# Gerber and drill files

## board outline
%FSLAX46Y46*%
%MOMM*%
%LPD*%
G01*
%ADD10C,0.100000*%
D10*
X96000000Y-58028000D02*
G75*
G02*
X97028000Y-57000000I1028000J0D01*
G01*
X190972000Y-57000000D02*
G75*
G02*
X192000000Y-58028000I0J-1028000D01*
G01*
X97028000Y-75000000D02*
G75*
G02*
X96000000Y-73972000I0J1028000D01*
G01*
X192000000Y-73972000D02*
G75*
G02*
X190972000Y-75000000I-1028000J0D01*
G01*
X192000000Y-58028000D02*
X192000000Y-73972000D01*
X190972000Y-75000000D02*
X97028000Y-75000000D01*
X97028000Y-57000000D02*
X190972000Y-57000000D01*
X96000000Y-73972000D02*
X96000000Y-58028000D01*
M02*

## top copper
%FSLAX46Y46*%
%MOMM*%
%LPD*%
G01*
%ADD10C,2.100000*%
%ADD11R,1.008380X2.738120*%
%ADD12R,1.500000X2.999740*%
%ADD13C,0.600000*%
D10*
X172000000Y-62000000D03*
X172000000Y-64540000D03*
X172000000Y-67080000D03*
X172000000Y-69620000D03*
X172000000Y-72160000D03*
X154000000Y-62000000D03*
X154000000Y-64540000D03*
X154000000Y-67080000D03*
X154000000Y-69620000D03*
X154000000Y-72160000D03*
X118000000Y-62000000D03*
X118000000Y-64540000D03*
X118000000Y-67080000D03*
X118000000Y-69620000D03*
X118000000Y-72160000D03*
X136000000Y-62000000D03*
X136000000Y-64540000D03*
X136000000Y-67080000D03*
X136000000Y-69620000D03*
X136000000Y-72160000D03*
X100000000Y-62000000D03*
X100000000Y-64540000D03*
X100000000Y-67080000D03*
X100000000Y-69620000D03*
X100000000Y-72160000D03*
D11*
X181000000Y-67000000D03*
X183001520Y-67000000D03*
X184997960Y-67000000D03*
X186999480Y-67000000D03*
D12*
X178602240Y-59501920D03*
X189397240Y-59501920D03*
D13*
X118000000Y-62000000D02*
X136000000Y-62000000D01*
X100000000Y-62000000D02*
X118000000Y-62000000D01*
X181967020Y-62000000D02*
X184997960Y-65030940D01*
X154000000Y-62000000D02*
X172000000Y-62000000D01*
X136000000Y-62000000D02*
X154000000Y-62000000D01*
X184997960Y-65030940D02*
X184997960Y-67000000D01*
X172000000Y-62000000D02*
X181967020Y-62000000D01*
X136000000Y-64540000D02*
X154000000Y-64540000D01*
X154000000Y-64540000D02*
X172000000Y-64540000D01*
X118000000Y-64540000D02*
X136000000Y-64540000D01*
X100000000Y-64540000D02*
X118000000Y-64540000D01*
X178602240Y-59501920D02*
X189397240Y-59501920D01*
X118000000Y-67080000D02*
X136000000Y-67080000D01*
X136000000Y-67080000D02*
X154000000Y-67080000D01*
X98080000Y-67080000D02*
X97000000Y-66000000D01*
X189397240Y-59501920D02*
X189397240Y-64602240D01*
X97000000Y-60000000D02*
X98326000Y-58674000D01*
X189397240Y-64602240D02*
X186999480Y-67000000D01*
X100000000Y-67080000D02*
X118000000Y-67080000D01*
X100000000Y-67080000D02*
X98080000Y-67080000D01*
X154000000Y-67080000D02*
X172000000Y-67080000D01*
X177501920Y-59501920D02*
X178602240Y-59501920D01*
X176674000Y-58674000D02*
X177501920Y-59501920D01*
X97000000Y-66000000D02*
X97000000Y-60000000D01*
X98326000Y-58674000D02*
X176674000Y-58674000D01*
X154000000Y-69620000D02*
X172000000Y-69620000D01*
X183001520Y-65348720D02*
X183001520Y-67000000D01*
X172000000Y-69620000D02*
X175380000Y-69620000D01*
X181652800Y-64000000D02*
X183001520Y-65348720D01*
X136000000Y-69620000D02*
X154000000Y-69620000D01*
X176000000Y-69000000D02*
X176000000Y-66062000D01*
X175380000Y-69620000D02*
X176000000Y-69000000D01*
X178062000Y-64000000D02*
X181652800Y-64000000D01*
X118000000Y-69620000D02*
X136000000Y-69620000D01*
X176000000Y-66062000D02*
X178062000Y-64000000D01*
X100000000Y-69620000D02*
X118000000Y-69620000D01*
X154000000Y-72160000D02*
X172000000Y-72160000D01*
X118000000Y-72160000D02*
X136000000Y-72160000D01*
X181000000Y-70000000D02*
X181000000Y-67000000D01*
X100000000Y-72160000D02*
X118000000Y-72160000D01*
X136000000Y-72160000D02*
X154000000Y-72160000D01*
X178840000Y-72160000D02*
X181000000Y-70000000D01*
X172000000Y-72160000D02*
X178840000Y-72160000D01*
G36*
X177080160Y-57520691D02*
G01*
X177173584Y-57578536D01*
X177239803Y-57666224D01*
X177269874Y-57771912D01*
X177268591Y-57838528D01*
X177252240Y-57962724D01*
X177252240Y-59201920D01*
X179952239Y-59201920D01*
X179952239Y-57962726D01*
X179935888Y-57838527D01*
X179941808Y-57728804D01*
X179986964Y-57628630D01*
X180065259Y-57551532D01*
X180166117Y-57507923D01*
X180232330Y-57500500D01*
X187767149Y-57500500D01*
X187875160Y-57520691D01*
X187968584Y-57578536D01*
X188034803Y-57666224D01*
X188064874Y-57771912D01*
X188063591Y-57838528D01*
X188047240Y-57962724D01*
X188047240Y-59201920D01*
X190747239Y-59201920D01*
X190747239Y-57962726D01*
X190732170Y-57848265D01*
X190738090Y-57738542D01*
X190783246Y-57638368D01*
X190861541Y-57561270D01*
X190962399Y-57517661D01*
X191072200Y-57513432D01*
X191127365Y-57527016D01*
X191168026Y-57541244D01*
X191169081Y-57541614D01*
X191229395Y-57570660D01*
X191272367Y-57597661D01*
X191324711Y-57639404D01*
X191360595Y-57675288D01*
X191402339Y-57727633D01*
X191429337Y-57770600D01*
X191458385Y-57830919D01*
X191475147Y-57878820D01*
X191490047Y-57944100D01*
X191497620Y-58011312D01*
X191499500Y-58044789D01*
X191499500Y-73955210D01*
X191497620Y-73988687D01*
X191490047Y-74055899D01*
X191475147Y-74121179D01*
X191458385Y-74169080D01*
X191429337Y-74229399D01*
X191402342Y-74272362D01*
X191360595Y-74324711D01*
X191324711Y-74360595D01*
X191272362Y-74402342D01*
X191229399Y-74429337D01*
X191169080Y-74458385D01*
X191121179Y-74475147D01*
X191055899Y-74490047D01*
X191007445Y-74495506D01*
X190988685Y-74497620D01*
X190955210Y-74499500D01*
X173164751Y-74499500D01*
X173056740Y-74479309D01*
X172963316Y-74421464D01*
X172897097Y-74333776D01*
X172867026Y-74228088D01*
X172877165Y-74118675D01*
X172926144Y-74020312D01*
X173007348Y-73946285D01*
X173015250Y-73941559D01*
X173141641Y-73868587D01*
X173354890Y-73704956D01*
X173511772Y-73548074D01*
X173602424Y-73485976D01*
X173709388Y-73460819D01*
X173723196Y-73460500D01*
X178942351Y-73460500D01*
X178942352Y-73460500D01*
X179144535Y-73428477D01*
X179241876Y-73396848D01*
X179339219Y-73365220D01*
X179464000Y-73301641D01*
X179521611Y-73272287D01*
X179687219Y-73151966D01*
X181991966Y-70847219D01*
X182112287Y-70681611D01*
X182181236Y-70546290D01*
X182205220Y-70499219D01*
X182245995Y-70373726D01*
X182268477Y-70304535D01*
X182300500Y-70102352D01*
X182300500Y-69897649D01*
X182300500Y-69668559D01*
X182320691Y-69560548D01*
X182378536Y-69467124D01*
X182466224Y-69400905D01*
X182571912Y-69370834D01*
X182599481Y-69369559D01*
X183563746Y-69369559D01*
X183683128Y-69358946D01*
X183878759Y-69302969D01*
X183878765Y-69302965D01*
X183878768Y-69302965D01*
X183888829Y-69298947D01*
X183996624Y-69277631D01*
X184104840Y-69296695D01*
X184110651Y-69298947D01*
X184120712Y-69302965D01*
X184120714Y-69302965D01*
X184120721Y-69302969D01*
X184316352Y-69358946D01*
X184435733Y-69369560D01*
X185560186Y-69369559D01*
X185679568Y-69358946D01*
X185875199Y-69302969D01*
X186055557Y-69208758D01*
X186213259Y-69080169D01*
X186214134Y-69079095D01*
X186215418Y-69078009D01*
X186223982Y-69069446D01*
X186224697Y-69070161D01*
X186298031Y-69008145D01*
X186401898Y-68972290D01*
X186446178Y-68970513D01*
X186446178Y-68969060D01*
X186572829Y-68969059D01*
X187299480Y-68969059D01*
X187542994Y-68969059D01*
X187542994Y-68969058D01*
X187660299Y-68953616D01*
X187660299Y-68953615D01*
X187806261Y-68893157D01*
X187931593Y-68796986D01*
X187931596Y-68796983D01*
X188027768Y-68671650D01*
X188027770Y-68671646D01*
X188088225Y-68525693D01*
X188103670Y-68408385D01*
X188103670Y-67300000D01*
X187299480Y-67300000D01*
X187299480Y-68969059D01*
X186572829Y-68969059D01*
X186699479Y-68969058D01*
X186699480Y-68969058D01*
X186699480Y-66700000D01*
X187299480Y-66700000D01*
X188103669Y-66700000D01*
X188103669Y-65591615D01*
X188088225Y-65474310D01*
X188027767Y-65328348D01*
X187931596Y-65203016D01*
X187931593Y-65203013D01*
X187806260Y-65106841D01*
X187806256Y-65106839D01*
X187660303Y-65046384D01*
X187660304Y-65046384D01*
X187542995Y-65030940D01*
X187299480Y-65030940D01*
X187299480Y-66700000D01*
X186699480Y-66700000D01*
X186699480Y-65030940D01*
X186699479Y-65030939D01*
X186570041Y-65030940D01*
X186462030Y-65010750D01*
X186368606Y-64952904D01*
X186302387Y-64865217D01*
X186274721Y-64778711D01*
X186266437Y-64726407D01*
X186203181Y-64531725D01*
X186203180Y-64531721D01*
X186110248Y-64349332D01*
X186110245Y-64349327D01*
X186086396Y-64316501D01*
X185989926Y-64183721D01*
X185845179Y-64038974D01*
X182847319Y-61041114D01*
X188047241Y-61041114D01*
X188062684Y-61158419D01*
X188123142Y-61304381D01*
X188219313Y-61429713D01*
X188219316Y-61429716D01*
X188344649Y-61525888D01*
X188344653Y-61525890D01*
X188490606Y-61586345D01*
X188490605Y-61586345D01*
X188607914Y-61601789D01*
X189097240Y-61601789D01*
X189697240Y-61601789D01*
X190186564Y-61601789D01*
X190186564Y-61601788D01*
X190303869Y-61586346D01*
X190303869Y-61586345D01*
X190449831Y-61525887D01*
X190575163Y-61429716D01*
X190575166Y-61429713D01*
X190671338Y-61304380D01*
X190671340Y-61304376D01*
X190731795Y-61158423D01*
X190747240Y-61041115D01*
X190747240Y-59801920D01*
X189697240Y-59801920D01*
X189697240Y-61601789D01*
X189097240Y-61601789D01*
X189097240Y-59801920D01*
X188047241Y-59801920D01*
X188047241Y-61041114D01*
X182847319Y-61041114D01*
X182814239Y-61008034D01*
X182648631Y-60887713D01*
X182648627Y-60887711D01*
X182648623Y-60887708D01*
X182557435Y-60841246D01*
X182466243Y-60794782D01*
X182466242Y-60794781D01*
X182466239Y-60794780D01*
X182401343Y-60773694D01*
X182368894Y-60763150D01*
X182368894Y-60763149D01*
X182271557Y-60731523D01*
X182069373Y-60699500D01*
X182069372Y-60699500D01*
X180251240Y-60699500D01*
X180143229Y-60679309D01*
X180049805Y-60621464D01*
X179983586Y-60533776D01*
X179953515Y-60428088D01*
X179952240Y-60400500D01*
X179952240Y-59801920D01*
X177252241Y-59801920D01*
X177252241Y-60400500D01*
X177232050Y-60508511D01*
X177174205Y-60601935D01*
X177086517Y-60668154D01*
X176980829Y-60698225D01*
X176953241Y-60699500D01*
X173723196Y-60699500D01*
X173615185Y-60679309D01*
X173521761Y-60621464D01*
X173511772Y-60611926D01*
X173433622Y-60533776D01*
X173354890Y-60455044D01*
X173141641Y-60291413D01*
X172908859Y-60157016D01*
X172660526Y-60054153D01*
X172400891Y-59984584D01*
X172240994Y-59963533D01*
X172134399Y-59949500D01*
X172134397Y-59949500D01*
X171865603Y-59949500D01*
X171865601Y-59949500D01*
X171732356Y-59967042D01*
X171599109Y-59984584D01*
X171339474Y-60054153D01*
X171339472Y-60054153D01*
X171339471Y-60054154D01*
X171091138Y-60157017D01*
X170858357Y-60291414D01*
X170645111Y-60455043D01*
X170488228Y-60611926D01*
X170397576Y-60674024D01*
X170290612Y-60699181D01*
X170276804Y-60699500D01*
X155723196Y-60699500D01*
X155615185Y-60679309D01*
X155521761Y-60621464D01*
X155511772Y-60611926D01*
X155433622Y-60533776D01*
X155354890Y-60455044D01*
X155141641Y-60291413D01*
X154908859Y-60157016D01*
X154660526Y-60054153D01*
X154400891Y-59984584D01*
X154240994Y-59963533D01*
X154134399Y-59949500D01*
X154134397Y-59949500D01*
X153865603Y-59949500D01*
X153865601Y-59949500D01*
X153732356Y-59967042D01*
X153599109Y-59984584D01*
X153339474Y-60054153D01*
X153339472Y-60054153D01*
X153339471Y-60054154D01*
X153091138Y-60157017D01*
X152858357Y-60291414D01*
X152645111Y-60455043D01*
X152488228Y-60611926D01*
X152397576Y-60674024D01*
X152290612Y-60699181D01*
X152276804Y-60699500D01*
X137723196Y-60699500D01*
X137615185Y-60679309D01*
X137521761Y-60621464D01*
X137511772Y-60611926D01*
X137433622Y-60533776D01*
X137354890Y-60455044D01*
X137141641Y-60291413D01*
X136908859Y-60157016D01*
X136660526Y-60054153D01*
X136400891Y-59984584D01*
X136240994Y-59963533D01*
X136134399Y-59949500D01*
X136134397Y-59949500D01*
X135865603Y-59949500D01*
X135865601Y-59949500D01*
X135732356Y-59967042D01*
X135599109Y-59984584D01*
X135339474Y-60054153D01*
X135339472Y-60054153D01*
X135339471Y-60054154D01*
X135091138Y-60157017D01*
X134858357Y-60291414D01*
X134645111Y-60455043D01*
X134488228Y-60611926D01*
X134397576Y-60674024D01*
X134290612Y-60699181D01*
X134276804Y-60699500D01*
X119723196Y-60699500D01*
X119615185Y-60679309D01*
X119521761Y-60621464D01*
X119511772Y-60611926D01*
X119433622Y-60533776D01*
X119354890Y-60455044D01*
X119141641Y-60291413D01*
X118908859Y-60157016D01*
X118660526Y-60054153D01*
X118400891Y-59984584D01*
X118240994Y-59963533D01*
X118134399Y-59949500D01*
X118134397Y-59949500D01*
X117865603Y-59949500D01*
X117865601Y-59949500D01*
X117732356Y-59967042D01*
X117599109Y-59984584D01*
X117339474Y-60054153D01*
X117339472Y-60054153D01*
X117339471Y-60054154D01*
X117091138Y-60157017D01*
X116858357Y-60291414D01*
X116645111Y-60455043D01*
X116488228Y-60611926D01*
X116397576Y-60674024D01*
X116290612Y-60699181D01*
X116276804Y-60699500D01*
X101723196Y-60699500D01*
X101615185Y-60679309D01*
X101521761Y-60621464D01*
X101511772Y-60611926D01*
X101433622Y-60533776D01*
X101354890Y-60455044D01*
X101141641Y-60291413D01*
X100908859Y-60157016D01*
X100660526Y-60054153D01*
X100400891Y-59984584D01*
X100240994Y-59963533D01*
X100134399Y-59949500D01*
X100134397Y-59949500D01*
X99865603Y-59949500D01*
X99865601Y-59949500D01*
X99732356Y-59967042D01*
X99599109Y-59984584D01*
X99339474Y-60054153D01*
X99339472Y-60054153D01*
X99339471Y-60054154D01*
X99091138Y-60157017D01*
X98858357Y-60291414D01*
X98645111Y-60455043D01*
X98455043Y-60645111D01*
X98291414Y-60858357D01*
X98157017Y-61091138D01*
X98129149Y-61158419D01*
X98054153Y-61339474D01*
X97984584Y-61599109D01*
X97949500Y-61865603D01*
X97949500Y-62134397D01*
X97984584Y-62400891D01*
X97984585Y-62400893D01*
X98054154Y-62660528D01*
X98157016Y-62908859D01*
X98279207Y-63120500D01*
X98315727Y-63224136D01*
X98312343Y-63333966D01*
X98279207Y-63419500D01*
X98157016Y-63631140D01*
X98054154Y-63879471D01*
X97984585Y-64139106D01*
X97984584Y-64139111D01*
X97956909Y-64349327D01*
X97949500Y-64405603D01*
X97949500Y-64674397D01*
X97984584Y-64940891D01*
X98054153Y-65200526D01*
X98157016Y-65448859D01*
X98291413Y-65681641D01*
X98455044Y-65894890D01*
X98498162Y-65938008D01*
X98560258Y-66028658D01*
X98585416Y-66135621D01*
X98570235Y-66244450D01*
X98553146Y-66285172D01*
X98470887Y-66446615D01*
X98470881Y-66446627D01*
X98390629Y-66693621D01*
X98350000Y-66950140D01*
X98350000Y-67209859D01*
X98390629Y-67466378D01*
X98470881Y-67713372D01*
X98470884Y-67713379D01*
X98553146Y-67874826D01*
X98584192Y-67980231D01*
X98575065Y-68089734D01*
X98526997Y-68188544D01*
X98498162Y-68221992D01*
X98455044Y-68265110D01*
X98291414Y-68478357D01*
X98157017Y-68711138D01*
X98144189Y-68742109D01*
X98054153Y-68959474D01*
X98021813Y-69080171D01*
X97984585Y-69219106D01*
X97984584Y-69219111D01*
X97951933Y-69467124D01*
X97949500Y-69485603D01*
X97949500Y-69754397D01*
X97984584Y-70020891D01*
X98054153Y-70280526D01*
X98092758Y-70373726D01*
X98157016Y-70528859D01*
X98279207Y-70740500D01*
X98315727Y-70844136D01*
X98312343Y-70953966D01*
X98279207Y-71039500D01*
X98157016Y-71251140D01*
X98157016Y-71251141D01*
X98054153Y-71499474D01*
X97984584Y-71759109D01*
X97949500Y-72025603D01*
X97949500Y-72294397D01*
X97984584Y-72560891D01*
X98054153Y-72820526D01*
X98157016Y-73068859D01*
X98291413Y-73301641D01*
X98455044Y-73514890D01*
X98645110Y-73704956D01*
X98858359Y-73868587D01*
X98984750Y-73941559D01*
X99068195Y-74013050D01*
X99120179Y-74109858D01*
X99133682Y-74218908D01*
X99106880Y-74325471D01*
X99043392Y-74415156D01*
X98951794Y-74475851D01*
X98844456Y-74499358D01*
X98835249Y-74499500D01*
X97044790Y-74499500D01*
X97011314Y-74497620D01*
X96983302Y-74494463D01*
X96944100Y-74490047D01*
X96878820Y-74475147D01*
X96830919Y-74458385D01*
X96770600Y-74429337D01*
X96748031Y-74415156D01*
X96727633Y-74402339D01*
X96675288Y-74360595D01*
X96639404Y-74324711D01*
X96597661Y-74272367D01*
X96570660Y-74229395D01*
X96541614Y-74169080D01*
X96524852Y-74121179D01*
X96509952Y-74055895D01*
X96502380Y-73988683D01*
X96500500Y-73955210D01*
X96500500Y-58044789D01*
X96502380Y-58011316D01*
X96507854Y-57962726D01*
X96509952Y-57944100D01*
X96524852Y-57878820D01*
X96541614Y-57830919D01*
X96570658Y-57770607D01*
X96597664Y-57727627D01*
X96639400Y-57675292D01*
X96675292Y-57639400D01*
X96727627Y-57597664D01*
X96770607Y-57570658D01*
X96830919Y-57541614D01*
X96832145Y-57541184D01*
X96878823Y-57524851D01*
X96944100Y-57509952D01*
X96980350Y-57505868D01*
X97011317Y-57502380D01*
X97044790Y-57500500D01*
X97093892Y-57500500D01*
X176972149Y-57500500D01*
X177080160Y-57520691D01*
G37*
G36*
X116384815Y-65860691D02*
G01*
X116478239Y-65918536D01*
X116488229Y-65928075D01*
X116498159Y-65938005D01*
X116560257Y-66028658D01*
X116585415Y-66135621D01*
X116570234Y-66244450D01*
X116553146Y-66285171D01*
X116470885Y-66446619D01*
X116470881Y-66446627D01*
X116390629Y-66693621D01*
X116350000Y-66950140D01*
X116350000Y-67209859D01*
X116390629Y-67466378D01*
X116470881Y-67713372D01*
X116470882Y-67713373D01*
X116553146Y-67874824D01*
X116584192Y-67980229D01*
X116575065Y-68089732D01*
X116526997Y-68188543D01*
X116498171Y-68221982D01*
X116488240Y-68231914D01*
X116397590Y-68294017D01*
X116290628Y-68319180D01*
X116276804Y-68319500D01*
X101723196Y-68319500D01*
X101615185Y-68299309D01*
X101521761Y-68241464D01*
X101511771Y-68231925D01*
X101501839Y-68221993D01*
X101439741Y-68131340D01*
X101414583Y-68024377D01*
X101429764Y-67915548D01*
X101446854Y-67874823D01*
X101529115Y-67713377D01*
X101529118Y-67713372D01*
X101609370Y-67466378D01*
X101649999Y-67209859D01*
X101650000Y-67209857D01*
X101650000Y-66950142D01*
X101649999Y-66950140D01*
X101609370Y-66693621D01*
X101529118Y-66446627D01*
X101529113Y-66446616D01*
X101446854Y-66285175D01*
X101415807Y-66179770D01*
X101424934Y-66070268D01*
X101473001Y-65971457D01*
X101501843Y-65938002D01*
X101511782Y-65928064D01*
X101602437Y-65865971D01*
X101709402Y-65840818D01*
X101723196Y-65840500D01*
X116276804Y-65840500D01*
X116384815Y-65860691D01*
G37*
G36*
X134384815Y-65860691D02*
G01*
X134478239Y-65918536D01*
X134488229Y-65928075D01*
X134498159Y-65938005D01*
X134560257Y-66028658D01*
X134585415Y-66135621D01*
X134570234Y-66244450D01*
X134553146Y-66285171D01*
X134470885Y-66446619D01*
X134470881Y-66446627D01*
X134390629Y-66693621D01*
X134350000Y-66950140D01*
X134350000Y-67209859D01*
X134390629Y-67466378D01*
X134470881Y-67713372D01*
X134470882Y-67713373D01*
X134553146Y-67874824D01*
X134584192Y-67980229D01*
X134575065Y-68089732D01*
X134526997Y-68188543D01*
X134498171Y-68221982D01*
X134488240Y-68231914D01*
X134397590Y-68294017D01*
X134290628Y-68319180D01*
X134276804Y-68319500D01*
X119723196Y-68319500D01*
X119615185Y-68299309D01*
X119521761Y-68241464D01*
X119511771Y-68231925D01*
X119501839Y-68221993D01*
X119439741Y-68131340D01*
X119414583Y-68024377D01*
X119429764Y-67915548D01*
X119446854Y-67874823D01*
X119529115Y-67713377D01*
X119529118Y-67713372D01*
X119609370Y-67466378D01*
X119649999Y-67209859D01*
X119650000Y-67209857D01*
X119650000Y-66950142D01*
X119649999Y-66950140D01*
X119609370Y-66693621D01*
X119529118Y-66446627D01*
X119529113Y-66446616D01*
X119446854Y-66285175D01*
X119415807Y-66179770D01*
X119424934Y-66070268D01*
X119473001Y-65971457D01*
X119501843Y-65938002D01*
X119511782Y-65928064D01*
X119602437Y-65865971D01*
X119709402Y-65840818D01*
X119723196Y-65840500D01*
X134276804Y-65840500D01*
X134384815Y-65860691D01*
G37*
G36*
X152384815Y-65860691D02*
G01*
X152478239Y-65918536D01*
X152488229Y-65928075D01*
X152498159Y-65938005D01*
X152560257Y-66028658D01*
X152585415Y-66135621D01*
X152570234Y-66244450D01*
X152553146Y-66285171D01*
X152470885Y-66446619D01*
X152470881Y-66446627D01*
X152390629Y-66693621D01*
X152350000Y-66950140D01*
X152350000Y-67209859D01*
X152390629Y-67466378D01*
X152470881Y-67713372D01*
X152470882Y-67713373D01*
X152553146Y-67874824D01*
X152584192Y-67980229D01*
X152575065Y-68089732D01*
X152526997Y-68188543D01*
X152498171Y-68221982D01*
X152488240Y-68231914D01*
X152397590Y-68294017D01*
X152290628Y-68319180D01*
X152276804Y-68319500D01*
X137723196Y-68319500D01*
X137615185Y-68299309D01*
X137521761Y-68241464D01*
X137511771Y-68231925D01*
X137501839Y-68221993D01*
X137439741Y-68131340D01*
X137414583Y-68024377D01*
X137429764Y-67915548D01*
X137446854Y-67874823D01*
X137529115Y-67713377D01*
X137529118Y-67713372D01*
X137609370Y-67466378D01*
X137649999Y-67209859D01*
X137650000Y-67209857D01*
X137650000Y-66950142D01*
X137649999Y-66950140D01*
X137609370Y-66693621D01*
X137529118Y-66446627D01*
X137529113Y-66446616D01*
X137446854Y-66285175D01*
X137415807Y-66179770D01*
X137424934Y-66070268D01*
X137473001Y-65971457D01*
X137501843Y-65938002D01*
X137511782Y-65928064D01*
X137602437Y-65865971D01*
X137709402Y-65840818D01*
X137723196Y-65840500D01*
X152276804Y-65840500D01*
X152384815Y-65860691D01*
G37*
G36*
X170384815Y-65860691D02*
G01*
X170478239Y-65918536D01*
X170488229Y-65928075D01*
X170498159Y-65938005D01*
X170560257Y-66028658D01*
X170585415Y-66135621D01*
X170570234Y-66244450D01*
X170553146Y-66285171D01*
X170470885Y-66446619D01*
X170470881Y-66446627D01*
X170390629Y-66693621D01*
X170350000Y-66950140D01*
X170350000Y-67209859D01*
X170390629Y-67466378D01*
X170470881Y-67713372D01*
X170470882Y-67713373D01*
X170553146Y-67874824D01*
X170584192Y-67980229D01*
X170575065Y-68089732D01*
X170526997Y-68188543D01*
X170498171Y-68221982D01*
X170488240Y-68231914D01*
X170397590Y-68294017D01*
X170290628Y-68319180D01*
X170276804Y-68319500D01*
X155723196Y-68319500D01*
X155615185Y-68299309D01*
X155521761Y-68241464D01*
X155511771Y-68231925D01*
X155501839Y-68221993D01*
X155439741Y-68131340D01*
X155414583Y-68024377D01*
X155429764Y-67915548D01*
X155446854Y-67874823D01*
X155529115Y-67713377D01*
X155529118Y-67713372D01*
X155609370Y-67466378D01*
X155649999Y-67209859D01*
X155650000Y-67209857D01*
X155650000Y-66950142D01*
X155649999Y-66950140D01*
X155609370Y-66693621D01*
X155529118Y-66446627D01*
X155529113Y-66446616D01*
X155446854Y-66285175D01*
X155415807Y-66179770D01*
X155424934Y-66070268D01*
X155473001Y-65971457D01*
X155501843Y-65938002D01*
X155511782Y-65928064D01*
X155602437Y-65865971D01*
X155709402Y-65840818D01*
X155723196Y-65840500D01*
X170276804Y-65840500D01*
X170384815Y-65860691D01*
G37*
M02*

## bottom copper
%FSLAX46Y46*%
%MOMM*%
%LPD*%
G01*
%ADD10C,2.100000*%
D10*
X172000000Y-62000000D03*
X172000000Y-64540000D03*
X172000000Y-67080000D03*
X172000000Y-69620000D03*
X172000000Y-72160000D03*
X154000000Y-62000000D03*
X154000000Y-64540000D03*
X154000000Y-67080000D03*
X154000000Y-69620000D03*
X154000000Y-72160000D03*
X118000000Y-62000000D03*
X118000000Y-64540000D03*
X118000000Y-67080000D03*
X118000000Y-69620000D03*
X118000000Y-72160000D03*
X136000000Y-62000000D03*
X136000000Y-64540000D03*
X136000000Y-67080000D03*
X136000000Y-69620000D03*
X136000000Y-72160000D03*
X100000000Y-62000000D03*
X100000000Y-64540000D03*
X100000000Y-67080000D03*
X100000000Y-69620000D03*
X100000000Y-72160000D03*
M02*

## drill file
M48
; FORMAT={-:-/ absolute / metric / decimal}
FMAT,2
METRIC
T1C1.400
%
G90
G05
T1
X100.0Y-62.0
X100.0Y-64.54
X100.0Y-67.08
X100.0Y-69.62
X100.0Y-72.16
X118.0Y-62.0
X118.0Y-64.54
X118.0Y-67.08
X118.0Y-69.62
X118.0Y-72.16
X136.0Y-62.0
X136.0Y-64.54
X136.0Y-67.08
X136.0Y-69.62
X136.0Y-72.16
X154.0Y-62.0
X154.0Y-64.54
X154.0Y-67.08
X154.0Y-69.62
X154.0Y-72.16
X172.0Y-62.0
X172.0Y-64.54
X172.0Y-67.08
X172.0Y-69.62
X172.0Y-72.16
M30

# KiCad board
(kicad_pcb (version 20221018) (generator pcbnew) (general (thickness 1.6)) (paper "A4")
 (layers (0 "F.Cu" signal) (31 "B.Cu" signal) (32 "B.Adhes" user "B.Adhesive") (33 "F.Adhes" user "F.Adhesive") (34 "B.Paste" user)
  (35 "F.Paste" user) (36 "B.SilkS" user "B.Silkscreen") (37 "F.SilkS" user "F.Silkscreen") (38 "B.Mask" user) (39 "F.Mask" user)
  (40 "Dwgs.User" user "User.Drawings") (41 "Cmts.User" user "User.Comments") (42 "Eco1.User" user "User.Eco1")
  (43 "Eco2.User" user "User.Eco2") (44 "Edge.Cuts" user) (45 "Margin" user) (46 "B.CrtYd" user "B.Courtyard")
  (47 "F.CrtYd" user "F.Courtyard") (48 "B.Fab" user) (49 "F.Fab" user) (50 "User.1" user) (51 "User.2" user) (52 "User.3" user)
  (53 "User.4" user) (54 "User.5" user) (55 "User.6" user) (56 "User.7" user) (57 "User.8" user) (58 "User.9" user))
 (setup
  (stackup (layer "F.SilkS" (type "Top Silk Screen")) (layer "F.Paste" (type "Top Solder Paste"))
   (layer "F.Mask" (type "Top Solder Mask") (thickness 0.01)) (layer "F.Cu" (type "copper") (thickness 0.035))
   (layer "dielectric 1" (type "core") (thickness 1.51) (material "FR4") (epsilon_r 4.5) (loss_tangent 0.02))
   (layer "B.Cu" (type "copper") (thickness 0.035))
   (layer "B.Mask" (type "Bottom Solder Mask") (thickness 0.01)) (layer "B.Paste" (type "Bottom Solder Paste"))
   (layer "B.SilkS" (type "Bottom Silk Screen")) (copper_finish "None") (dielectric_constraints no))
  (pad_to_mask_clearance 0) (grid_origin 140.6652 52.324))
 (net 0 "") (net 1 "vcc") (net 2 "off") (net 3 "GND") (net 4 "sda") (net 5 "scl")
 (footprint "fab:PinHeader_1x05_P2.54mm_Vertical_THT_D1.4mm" (layer "F.Cu") (at 172 62)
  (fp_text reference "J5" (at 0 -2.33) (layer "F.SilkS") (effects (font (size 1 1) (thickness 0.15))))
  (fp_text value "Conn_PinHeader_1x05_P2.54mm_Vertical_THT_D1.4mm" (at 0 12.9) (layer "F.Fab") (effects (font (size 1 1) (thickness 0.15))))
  (pad "1" thru_hole circle (at 0 0) (size 2.1 2.1) (drill 1.4) (layers "*.Cu" "*.Mask") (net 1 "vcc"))
  (pad "2" thru_hole circle (at 0 2.54) (size 2.1 2.1) (drill 1.4) (layers "*.Cu" "*.Mask") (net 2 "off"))
  (pad "3" thru_hole circle (at 0 5.08) (size 2.1 2.1) (drill 1.4) (layers "*.Cu" "*.Mask") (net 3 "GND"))
  (pad "4" thru_hole circle (at 0 7.62) (size 2.1 2.1) (drill 1.4) (layers "*.Cu" "*.Mask") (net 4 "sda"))
  (pad "5" thru_hole circle (at 0 10.16) (size 2.1 2.1) (drill 1.4) (layers "*.Cu" "*.Mask") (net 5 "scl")))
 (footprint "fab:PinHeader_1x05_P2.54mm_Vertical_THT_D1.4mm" (layer "F.Cu") (at 154 62)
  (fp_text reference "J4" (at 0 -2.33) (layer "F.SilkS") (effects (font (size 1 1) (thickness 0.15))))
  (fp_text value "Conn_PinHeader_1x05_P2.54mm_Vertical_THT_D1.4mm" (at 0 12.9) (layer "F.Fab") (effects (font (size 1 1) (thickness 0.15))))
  (pad "1" thru_hole circle (at 0 0) (size 2.1 2.1) (drill 1.4) (layers "*.Cu" "*.Mask") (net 1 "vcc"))
  (pad "2" thru_hole circle (at 0 2.54) (size 2.1 2.1) (drill 1.4) (layers "*.Cu" "*.Mask") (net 2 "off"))
  (pad "3" thru_hole circle (at 0 5.08) (size 2.1 2.1) (drill 1.4) (layers "*.Cu" "*.Mask") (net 3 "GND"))
  (pad "4" thru_hole circle (at 0 7.62) (size 2.1 2.1) (drill 1.4) (layers "*.Cu" "*.Mask") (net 4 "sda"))
  (pad "5" thru_hole circle (at 0 10.16) (size 2.1 2.1) (drill 1.4) (layers "*.Cu" "*.Mask") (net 5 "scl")))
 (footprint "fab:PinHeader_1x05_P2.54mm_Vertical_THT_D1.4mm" (layer "F.Cu") (at 118 62)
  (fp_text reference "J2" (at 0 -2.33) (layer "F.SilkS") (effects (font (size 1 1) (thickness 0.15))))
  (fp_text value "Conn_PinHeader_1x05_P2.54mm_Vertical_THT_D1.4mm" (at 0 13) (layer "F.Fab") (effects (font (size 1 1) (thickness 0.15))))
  (pad "1" thru_hole circle (at 0 0) (size 2.1 2.1) (drill 1.4) (layers "*.Cu" "*.Mask") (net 1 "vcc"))
  (pad "2" thru_hole circle (at 0 2.54) (size 2.1 2.1) (drill 1.4) (layers "*.Cu" "*.Mask") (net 2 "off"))
  (pad "3" thru_hole circle (at 0 5.08) (size 2.1 2.1) (drill 1.4) (layers "*.Cu" "*.Mask") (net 3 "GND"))
  (pad "4" thru_hole circle (at 0 7.62) (size 2.1 2.1) (drill 1.4) (layers "*.Cu" "*.Mask") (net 4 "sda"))
  (pad "5" thru_hole circle (at 0 10.16) (size 2.1 2.1) (drill 1.4) (layers "*.Cu" "*.Mask") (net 5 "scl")))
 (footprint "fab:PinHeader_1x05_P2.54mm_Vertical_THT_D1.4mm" (layer "F.Cu") (at 136 62)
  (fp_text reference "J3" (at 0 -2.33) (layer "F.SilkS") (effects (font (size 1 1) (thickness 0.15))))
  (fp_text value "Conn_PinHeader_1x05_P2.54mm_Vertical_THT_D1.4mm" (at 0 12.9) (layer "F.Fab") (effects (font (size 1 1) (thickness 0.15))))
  (pad "1" thru_hole circle (at 0 0) (size 2.1 2.1) (drill 1.4) (layers "*.Cu" "*.Mask") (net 1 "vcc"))
  (pad "2" thru_hole circle (at 0 2.54) (size 2.1 2.1) (drill 1.4) (layers "*.Cu" "*.Mask") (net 2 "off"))
  (pad "3" thru_hole circle (at 0 5.08) (size 2.1 2.1) (drill 1.4) (layers "*.Cu" "*.Mask") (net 3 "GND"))
  (pad "4" thru_hole circle (at 0 7.62) (size 2.1 2.1) (drill 1.4) (layers "*.Cu" "*.Mask") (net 4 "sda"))
  (pad "5" thru_hole circle (at 0 10.16) (size 2.1 2.1) (drill 1.4) (layers "*.Cu" "*.Mask") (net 5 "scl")))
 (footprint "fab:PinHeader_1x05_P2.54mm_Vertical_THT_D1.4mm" (layer "F.Cu") (at 100 62)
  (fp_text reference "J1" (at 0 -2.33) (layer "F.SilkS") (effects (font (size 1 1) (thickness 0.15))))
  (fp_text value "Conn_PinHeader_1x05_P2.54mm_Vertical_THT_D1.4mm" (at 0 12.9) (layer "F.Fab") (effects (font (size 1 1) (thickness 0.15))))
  (pad "1" thru_hole circle (at 0 0) (size 2.1 2.1) (drill 1.4) (layers "*.Cu" "*.Mask") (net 1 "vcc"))
  (pad "2" thru_hole circle (at 0 2.54) (size 2.1 2.1) (drill 1.4) (layers "*.Cu" "*.Mask") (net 2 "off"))
  (pad "3" thru_hole circle (at 0 5.08) (size 2.1 2.1) (drill 1.4) (layers "*.Cu" "*.Mask") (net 3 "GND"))
  (pad "4" thru_hole circle (at 0 7.62) (size 2.1 2.1) (drill 1.4) (layers "*.Cu" "*.Mask") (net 4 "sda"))
  (pad "5" thru_hole circle (at 0 10.16) (size 2.1 2.1) (drill 1.4) (layers "*.Cu" "*.Mask") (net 5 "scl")))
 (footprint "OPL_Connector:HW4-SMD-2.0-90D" (layer "F.Cu") (at 183.99974 62.2003)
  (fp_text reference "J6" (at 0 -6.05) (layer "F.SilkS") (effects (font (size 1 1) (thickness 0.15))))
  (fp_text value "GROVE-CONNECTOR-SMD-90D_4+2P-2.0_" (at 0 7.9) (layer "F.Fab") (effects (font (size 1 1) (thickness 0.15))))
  (pad "1" smd rect (at -2.99974 4.7997 90) (size 2.73812 1.00838) (layers "F.Cu" "F.Paste" "F.Mask") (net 5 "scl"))
  (pad "2" smd rect (at -0.99822 4.7997 90) (size 2.73812 1.00838) (layers "F.Cu" "F.Paste" "F.Mask") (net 4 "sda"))
  (pad "3" smd rect (at 0.99822 4.7997 90) (size 2.73812 1.00838) (layers "F.Cu" "F.Paste" "F.Mask") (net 1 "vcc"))
  (pad "4" smd rect (at 2.99974 4.7997 90) (size 2.73812 1.00838) (layers "F.Cu" "F.Paste" "F.Mask") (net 3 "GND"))
  (pad "5" smd rect (at -5.3975 -2.69838 90) (size 2.99974 1.5) (layers "F.Cu" "F.Paste" "F.Mask") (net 3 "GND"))
  (pad "6" smd rect (at 5.3975 -2.69838 90) (size 2.99974 1.5) (layers "F.Cu" "F.Paste" "F.Mask") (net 3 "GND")))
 (gr_arc (start 96 58.028) (mid 96.301094 57.301094) (end 97.028 57) (stroke (width 0.1) (type default)) (layer "Edge.Cuts"))
 (gr_arc (start 190.972 57) (mid 191.698906 57.301094) (end 192 58.028) (stroke (width 0.1) (type default)) (layer "Edge.Cuts"))
 (gr_arc (start 97.028 75) (mid 96.301094 74.698906) (end 96 73.972) (stroke (width 0.1) (type default)) (layer "Edge.Cuts"))
 (gr_arc (start 192 73.972) (mid 191.698906 74.698906) (end 190.972 75) (stroke (width 0.1) (type default)) (layer "Edge.Cuts"))
 (gr_line (start 192 58.028) (end 192 73.972) (stroke (width 0.1) (type default)) (layer "Edge.Cuts"))
 (gr_line (start 190.972 75) (end 97.028 75) (stroke (width 0.1) (type default)) (layer "Edge.Cuts"))
 (gr_line (start 97.028 57) (end 190.972 57) (stroke (width 0.1) (type default)) (layer "Edge.Cuts"))
 (gr_line (start 96 73.972) (end 96 58.028) (stroke (width 0.1) (type default)) (layer "Edge.Cuts"))
 (segment (start 118 62) (end 136 62) (width 0.6) (layer "F.Cu") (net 1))
 (segment (start 100 62) (end 118 62) (width 0.6) (layer "F.Cu") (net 1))
 (segment (start 181.96702 62) (end 184.99796 65.03094) (width 0.6) (layer "F.Cu") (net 1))
 (segment (start 154 62) (end 172 62) (width 0.6) (layer "F.Cu") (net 1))
 (segment (start 136 62) (end 154 62) (width 0.6) (layer "F.Cu") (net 1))
 (segment (start 184.99796 65.03094) (end 184.99796 67) (width 0.6) (layer "F.Cu") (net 1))
 (segment (start 172 62) (end 181.96702 62) (width 0.6) (layer "F.Cu") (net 1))
 (segment (start 136 64.54) (end 154 64.54) (width 0.6) (layer "F.Cu") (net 2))
 (segment (start 154 64.54) (end 172 64.54) (width 0.6) (layer "F.Cu") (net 2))
 (segment (start 118 64.54) (end 136 64.54) (width 0.6) (layer "F.Cu") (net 2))
 (segment (start 100 64.54) (end 118 64.54) (width 0.6) (layer "F.Cu") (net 2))
 (segment (start 178.60224 59.50192) (end 189.39724 59.50192) (width 0.6) (layer "F.Cu") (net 3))
 (segment (start 118 67.08) (end 136 67.08) (width 0.6) (layer "F.Cu") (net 3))
 (segment (start 136 67.08) (end 154 67.08) (width 0.6) (layer "F.Cu") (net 3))
 (segment (start 98.08 67.08) (end 97 66) (width 0.6) (layer "F.Cu") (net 3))
 (segment (start 189.39724 59.50192) (end 189.39724 64.60224) (width 0.6) (layer "F.Cu") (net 3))
 (segment (start 97 60) (end 98.326 58.674) (width 0.6) (layer "F.Cu") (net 3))
 (segment (start 189.39724 64.60224) (end 186.99948 67) (width 0.6) (layer "F.Cu") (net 3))
 (segment (start 100 67.08) (end 118 67.08) (width 0.6) (layer "F.Cu") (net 3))
 (segment (start 100 67.08) (end 98.08 67.08) (width 0.6) (layer "F.Cu") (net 3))
 (segment (start 154 67.08) (end 172 67.08) (width 0.6) (layer "F.Cu") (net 3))
 (segment (start 177.50192 59.50192) (end 178.60224 59.50192) (width 0.6) (layer "F.Cu") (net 3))
 (segment (start 176.674 58.674) (end 177.50192 59.50192) (width 0.6) (layer "F.Cu") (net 3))
 (segment (start 97 66) (end 97 60) (width 0.6) (layer "F.Cu") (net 3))
 (segment (start 98.326 58.674) (end 176.674 58.674) (width 0.6) (layer "F.Cu") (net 3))
 (segment (start 154 69.62) (end 172 69.62) (width 0.6) (layer "F.Cu") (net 4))
 (segment (start 183.00152 65.34872) (end 183.00152 67) (width 0.6) (layer "F.Cu") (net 4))
 (segment (start 172 69.62) (end 175.38 69.62) (width 0.6) (layer "F.Cu") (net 4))
 (segment (start 181.6528 64) (end 183.00152 65.34872) (width 0.6) (layer "F.Cu") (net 4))
 (segment (start 136 69.62) (end 154 69.62) (width 0.6) (layer "F.Cu") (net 4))
 (segment (start 176 69) (end 176 66.062) (width 0.6) (layer "F.Cu") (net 4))
 (segment (start 175.38 69.62) (end 176 69) (width 0.6) (layer "F.Cu") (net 4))
 (segment (start 178.062 64) (end 181.6528 64) (width 0.6) (layer "F.Cu") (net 4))
 (segment (start 118 69.62) (end 136 69.62) (width 0.6) (layer "F.Cu") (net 4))
 (segment (start 176 66.062) (end 178.062 64) (width 0.6) (layer "F.Cu") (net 4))
 (segment (start 100 69.62) (end 118 69.62) (width 0.6) (layer "F.Cu") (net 4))
 (segment (start 154 72.16) (end 172 72.16) (width 0.6) (layer "F.Cu") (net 5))
 (segment (start 118 72.16) (end 136 72.16) (width 0.6) (layer "F.Cu") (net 5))
 (segment (start 181 70) (end 181 67) (width 0.6) (layer "F.Cu") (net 5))
 (segment (start 100 72.16) (end 118 72.16) (width 0.6) (layer "F.Cu") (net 5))
 (segment (start 136 72.16) (end 154 72.16) (width 0.6) (layer "F.Cu") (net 5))
 (segment (start 178.84 72.16) (end 181 70) (width 0.6) (layer "F.Cu") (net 5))
 (segment (start 172 72.16) (end 178.84 72.16) (width 0.6) (layer "F.Cu") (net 5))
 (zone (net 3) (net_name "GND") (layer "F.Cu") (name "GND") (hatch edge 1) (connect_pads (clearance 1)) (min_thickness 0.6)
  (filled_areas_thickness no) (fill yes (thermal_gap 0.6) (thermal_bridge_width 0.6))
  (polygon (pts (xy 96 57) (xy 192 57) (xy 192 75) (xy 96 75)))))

